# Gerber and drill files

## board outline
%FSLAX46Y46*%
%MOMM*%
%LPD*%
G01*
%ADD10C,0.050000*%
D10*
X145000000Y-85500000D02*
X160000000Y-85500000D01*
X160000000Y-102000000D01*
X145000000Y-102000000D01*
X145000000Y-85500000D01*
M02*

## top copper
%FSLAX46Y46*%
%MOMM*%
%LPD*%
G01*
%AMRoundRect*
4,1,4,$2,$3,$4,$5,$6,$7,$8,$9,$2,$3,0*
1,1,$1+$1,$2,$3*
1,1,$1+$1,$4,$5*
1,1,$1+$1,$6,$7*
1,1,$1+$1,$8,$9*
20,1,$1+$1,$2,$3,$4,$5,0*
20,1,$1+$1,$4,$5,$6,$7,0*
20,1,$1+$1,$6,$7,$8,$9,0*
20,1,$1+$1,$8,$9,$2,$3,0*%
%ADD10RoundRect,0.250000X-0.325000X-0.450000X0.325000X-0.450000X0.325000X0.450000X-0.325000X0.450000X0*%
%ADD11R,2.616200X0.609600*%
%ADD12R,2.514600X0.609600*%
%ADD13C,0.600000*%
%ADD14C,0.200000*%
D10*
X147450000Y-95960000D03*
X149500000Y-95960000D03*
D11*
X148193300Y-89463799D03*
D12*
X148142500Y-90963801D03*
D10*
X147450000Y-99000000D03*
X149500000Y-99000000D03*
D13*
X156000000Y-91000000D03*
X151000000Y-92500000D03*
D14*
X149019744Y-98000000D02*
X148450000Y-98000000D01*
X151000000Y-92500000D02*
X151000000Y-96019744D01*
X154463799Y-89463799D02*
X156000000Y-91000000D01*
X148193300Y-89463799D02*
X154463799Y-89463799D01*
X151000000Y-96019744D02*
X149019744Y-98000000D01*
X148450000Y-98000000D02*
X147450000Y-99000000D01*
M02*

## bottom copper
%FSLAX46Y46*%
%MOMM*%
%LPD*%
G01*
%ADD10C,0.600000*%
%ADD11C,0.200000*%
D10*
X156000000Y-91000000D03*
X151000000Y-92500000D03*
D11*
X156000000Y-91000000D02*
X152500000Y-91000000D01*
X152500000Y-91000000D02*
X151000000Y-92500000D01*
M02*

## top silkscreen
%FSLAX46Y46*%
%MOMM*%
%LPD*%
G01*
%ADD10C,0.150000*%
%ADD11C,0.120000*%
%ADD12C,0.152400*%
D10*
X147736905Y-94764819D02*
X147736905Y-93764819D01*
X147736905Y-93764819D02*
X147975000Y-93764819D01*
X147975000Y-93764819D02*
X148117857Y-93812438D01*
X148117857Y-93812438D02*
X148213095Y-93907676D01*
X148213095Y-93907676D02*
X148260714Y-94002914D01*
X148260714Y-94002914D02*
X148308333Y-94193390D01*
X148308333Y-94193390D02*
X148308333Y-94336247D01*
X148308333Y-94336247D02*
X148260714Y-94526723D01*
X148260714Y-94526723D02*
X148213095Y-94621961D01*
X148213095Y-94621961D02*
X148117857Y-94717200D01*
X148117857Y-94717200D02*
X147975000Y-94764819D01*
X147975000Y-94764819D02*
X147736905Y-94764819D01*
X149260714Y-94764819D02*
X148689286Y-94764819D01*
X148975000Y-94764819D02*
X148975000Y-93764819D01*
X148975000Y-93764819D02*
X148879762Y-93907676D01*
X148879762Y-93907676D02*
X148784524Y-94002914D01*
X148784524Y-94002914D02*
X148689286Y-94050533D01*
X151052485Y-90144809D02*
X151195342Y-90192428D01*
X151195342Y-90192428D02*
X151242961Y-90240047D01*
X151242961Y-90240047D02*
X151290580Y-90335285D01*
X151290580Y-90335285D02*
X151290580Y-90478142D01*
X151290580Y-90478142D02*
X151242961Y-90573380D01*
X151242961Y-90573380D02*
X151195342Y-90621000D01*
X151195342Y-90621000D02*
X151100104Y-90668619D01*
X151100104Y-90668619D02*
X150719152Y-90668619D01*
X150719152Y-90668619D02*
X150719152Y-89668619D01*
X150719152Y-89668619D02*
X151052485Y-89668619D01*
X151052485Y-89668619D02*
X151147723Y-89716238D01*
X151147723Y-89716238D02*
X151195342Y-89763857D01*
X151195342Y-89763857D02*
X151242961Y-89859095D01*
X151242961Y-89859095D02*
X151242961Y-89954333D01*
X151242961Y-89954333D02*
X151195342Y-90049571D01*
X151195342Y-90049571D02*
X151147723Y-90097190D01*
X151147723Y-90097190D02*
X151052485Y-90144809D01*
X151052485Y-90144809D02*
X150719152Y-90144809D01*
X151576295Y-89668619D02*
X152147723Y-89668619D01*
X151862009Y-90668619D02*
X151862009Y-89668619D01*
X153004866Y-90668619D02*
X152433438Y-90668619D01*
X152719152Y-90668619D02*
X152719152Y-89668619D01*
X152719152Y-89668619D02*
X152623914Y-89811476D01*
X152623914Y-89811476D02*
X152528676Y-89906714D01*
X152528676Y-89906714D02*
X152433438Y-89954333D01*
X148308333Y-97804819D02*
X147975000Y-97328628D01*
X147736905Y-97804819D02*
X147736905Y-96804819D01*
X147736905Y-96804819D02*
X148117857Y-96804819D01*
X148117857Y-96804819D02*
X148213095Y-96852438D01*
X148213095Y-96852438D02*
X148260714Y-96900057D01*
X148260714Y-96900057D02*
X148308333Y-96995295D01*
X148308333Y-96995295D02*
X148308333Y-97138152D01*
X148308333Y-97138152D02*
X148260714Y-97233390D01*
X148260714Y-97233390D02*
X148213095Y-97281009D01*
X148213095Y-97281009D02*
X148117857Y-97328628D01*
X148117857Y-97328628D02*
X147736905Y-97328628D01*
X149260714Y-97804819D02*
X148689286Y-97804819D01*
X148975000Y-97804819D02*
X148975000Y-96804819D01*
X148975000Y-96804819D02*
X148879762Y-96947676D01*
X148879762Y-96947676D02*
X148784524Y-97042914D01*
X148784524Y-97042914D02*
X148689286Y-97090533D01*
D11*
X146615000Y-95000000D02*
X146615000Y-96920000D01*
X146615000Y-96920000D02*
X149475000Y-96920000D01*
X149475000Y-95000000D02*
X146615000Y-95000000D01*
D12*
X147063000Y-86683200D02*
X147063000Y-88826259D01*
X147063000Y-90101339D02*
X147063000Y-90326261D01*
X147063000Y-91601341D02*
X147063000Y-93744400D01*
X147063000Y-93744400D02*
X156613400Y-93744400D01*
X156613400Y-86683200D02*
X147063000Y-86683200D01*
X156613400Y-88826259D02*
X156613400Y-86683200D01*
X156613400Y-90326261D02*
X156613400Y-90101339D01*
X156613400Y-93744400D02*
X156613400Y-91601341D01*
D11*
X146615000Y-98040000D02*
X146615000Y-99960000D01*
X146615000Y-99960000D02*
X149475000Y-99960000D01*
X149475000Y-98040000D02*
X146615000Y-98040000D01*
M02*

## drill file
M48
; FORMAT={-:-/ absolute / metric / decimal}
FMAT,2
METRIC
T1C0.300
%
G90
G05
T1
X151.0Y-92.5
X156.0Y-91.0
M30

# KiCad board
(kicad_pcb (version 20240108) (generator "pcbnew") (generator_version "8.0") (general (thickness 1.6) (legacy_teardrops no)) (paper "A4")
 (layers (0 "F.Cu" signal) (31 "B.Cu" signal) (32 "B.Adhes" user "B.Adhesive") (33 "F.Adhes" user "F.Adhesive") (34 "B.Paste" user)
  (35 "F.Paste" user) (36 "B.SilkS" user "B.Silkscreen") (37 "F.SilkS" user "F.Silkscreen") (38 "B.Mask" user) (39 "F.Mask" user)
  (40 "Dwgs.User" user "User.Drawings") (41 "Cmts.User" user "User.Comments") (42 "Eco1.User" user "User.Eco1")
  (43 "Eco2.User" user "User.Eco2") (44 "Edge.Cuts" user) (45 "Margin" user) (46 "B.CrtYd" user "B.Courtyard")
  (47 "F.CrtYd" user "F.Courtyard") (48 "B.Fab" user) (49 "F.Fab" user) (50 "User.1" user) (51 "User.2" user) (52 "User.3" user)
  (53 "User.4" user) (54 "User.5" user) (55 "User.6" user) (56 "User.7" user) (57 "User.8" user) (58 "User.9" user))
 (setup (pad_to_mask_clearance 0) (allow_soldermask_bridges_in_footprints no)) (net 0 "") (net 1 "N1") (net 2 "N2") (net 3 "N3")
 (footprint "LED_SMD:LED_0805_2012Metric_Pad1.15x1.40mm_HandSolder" (layer "F.Cu") (at 148.475 95.96)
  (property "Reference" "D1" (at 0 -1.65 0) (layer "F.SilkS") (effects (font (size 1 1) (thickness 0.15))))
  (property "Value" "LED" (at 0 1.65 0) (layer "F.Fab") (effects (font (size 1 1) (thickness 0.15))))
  (fp_line (start -1.86 -0.96) (end -1.86 0.96) (stroke (width 0.12) (type solid)) (layer "F.SilkS"))
  (fp_line (start -1.86 0.96) (end 1 0.96) (stroke (width 0.12) (type solid)) (layer "F.SilkS"))
  (fp_line (start 1 -0.96) (end -1.86 -0.96) (stroke (width 0.12) (type solid)) (layer "F.SilkS"))
  (pad "1" smd roundrect (at -1.025 0) (size 1.15 1.4) (layers "F.Cu" "F.Paste" "F.Mask") (roundrect_rratio 0.217391) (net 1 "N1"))
  (pad "2" smd roundrect (at 1.025 0) (size 1.15 1.4) (layers "F.Cu" "F.Paste" "F.Mask") (roundrect_rratio 0.217391) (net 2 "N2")))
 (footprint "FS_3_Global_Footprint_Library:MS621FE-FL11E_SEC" (layer "F.Cu") (at 151.8382 90.2138)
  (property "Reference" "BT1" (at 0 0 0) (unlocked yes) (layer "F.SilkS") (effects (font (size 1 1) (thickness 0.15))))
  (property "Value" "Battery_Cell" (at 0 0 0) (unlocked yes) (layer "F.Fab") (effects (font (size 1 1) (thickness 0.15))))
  (fp_line (start -4.7752 -3.5306) (end -4.7752 -1.387541) (stroke (width 0.1524) (type solid)) (layer "F.SilkS"))
  (fp_line (start -4.7752 -0.112461) (end -4.7752 0.112461) (stroke (width 0.1524) (type solid)) (layer "F.SilkS"))
  (fp_line (start -4.7752 1.387541) (end -4.7752 3.5306) (stroke (width 0.1524) (type solid)) (layer "F.SilkS"))
  (fp_line (start -4.7752 3.5306) (end 4.7752 3.5306) (stroke (width 0.1524) (type solid)) (layer "F.SilkS"))
  (fp_line (start 4.7752 -3.5306) (end -4.7752 -3.5306) (stroke (width 0.1524) (type solid)) (layer "F.SilkS"))
  (fp_line (start 4.7752 -1.387541) (end 4.7752 -3.5306) (stroke (width 0.1524) (type solid)) (layer "F.SilkS"))
  (fp_line (start 4.7752 0.112461) (end 4.7752 -0.112461) (stroke (width 0.1524) (type solid)) (layer "F.SilkS"))
  (fp_line (start 4.7752 3.5306) (end 4.7752 1.387541) (stroke (width 0.1524) (type solid)) (layer "F.SilkS"))
  (pad "1" smd rect (at -3.6449 -0.750001) (size 2.6162 0.6096) (layers "F.Cu" "F.Paste" "F.Mask") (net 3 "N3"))
  (pad "2" smd rect (at -3.6957 0.750001) (size 2.5146 0.6096) (layers "F.Cu" "F.Paste" "F.Mask") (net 1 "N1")))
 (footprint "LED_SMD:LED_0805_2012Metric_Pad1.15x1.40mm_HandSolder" (layer "F.Cu") (at 148.475 99)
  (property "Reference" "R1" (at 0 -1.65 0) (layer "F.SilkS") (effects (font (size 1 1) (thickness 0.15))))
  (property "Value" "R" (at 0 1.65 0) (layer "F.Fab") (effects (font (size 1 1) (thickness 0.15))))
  (fp_line (start -1.86 -0.96) (end -1.86 0.96) (stroke (width 0.12) (type solid)) (layer "F.SilkS"))
  (fp_line (start -1.86 0.96) (end 1 0.96) (stroke (width 0.12) (type solid)) (layer "F.SilkS"))
  (fp_line (start 1 -0.96) (end -1.86 -0.96) (stroke (width 0.12) (type solid)) (layer "F.SilkS"))
  (pad "1" smd roundrect (at -1.025 0) (size 1.15 1.4) (layers "F.Cu" "F.Paste" "F.Mask") (roundrect_rratio 0.217391) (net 3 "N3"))
  (pad "2" smd roundrect (at 1.025 0) (size 1.15 1.4) (layers "F.Cu" "F.Paste" "F.Mask") (roundrect_rratio 0.217391) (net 2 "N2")))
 (gr_rect (start 145 85.5) (end 160 102) (stroke (width 0.05) (type default)) (fill none) (layer "Edge.Cuts"))
 (segment (start 149.019744 98) (end 148.45 98) (width 0.2) (layer "F.Cu") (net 3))
 (segment (start 151 92.5) (end 151 96.019744) (width 0.2) (layer "F.Cu") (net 3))
 (segment (start 154.463799 89.463799) (end 156 91) (width 0.2) (layer "F.Cu") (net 3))
 (segment (start 148.1933 89.463799) (end 154.463799 89.463799) (width 0.2) (layer "F.Cu") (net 3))
 (segment (start 151 96.019744) (end 149.019744 98) (width 0.2) (layer "F.Cu") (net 3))
 (segment (start 148.45 98) (end 147.45 99) (width 0.2) (layer "F.Cu") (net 3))
 (via (at 156 91) (size 0.6) (drill 0.3) (layers "F.Cu" "B.Cu") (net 3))
 (via (at 151 92.5) (size 0.6) (drill 0.3) (layers "F.Cu" "B.Cu") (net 3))
 (segment (start 156 91) (end 152.5 91) (width 0.2) (layer "B.Cu") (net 3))
 (segment (start 152.5 91) (end 151 92.5) (width 0.2) (layer "B.Cu") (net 3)))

